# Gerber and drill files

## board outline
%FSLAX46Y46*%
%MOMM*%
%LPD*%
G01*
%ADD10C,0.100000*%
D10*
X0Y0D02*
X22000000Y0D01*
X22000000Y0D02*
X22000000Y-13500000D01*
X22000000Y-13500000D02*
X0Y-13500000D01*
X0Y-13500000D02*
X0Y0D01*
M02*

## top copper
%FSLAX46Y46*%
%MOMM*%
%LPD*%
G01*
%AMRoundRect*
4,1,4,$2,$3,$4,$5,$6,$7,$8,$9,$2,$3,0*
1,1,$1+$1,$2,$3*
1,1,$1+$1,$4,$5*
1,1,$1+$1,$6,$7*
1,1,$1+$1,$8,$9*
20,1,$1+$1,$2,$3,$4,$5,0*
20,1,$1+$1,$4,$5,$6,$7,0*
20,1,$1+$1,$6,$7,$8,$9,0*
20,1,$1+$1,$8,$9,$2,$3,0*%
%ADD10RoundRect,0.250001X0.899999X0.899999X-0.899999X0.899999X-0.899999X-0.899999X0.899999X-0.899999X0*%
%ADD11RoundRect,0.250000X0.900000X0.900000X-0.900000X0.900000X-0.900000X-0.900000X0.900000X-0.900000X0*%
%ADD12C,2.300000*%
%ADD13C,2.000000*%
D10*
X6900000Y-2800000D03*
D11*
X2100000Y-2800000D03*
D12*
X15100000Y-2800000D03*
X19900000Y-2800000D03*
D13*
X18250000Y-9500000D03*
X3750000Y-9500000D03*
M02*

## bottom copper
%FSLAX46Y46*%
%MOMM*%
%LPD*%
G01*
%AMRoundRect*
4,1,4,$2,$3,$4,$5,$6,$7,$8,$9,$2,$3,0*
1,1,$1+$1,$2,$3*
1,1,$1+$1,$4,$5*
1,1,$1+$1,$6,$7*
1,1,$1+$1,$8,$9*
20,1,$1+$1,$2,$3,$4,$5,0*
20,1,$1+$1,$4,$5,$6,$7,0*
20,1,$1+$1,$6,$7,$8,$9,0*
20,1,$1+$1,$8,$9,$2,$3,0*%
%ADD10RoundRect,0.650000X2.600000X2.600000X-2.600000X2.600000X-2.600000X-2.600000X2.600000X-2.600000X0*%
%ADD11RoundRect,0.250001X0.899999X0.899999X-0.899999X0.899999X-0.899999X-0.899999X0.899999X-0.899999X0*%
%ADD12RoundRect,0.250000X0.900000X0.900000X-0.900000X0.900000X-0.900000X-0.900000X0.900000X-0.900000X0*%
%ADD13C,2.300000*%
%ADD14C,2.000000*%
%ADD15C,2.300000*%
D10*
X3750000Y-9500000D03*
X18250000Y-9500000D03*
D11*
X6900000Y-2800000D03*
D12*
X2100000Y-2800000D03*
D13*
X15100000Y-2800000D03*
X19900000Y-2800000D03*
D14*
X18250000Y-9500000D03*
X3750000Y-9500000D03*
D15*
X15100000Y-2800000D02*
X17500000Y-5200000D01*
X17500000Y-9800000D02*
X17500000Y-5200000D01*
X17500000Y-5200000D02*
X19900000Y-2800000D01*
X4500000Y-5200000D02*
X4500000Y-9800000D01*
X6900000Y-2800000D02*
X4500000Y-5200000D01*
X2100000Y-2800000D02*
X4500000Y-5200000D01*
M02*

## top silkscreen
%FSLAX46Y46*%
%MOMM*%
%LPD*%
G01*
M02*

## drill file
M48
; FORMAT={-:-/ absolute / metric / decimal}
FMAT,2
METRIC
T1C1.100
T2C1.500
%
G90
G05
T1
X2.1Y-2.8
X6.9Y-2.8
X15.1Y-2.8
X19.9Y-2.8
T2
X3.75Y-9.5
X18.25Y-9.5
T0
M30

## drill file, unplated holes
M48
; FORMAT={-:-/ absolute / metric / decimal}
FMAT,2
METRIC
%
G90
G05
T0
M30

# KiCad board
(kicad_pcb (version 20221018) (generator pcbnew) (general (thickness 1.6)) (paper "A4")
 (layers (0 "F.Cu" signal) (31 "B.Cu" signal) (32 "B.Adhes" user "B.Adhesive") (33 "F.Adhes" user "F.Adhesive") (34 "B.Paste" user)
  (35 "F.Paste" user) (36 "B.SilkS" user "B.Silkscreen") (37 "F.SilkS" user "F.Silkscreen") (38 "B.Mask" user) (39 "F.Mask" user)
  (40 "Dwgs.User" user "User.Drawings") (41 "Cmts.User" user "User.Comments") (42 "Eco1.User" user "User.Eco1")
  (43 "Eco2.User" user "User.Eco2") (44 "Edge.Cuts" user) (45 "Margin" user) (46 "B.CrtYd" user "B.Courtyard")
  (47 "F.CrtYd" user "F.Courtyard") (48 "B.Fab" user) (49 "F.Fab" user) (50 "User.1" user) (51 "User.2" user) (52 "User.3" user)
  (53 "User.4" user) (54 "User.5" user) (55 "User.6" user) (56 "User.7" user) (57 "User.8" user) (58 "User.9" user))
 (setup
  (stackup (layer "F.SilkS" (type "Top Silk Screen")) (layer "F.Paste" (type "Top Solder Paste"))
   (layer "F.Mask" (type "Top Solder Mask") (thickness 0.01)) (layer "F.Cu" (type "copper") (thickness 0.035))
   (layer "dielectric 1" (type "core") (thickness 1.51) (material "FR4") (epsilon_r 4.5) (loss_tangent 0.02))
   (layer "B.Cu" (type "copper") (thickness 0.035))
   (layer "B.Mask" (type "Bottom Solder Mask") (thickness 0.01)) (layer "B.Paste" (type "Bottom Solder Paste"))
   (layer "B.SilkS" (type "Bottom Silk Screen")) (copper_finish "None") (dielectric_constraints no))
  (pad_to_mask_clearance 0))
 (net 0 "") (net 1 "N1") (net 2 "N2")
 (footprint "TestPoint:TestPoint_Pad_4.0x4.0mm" (layer "B.Cu") (at 3.75 9.5 180)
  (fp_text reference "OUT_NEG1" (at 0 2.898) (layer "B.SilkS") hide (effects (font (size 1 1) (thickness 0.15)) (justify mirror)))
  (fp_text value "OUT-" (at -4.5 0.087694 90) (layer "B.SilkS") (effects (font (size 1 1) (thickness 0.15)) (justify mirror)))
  (pad "1" smd roundrect (at 0 0 180) (size 6.5 6.5) (layers "B.Cu" "B.Mask") (roundrect_rratio 0.1) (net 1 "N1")))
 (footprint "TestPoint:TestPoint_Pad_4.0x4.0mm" (layer "B.Cu") (at 18.25 9.5 180)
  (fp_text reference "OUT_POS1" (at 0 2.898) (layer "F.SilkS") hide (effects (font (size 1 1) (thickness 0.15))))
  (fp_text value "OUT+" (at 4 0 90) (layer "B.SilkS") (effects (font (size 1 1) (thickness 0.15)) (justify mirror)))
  (pad "1" smd roundrect (at 0 0 180) (size 6.5 6.5) (layers "B.Cu" "B.Mask") (roundrect_rratio 0.1) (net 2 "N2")))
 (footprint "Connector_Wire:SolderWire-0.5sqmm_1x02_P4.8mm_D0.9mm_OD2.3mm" (layer "B.Cu") (at 6.9 2.8 180)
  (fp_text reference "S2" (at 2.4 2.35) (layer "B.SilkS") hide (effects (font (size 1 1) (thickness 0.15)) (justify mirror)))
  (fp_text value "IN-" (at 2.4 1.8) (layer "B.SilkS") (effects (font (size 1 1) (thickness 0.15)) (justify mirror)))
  (pad "1" thru_hole roundrect (at 0 0 180) (size 2.3 2.3) (drill 1.1) (layers "*.Cu" "*.Mask") (roundrect_rratio 0.108696087) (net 1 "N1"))
  (pad "2" thru_hole roundrect (at 4.8 0 180) (size 2.3 2.3) (drill 1.1) (layers "*.Cu" "*.Mask") (roundrect_rratio 0.1086956522)
   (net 1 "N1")))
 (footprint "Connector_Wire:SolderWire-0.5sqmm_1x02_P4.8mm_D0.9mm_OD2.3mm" (layer "B.Cu") (at 19.9 2.8 180)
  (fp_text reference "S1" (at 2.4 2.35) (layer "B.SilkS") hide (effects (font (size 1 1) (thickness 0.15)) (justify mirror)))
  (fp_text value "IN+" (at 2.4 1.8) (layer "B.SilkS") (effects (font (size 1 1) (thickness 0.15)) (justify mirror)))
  (pad "1" thru_hole circle (at 0 0 180) (size 2.3 2.3) (drill 1.1) (layers "*.Cu" "*.Mask") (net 2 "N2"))
  (pad "2" thru_hole circle (at 4.8 0 180) (size 2.3 2.3) (drill 1.1) (layers "*.Cu" "*.Mask") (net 2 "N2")))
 (gr_rect (start 0 0) (end 22 13.5) (stroke (width 0.1) (type default)) (fill none) (layer "Edge.Cuts"))
 (via (at 18.25 9.5) (size 2) (drill 1.5) (layers "F.Cu" "B.Cu") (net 2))
 (segment (start 15.1 2.8) (end 17.5 5.2) (width 2.3) (layer "B.Cu") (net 2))
 (segment (start 17.5 9.8) (end 17.5 5.2) (width 2.3) (layer "B.Cu") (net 2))
 (segment (start 17.5 5.2) (end 19.9 2.8) (width 2.3) (layer "B.Cu") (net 2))
 (via (at 3.75 9.5) (size 2) (drill 1.5) (layers "F.Cu" "B.Cu") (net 1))
 (segment (start 4.5 5.2) (end 4.5 9.8) (width 2.3) (layer "B.Cu") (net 1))
 (segment (start 6.9 2.8) (end 4.5 5.2) (width 2.3) (layer "B.Cu") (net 1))
 (segment (start 2.1 2.8) (end 4.5 5.2) (width 2.3) (layer "B.Cu") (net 1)))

